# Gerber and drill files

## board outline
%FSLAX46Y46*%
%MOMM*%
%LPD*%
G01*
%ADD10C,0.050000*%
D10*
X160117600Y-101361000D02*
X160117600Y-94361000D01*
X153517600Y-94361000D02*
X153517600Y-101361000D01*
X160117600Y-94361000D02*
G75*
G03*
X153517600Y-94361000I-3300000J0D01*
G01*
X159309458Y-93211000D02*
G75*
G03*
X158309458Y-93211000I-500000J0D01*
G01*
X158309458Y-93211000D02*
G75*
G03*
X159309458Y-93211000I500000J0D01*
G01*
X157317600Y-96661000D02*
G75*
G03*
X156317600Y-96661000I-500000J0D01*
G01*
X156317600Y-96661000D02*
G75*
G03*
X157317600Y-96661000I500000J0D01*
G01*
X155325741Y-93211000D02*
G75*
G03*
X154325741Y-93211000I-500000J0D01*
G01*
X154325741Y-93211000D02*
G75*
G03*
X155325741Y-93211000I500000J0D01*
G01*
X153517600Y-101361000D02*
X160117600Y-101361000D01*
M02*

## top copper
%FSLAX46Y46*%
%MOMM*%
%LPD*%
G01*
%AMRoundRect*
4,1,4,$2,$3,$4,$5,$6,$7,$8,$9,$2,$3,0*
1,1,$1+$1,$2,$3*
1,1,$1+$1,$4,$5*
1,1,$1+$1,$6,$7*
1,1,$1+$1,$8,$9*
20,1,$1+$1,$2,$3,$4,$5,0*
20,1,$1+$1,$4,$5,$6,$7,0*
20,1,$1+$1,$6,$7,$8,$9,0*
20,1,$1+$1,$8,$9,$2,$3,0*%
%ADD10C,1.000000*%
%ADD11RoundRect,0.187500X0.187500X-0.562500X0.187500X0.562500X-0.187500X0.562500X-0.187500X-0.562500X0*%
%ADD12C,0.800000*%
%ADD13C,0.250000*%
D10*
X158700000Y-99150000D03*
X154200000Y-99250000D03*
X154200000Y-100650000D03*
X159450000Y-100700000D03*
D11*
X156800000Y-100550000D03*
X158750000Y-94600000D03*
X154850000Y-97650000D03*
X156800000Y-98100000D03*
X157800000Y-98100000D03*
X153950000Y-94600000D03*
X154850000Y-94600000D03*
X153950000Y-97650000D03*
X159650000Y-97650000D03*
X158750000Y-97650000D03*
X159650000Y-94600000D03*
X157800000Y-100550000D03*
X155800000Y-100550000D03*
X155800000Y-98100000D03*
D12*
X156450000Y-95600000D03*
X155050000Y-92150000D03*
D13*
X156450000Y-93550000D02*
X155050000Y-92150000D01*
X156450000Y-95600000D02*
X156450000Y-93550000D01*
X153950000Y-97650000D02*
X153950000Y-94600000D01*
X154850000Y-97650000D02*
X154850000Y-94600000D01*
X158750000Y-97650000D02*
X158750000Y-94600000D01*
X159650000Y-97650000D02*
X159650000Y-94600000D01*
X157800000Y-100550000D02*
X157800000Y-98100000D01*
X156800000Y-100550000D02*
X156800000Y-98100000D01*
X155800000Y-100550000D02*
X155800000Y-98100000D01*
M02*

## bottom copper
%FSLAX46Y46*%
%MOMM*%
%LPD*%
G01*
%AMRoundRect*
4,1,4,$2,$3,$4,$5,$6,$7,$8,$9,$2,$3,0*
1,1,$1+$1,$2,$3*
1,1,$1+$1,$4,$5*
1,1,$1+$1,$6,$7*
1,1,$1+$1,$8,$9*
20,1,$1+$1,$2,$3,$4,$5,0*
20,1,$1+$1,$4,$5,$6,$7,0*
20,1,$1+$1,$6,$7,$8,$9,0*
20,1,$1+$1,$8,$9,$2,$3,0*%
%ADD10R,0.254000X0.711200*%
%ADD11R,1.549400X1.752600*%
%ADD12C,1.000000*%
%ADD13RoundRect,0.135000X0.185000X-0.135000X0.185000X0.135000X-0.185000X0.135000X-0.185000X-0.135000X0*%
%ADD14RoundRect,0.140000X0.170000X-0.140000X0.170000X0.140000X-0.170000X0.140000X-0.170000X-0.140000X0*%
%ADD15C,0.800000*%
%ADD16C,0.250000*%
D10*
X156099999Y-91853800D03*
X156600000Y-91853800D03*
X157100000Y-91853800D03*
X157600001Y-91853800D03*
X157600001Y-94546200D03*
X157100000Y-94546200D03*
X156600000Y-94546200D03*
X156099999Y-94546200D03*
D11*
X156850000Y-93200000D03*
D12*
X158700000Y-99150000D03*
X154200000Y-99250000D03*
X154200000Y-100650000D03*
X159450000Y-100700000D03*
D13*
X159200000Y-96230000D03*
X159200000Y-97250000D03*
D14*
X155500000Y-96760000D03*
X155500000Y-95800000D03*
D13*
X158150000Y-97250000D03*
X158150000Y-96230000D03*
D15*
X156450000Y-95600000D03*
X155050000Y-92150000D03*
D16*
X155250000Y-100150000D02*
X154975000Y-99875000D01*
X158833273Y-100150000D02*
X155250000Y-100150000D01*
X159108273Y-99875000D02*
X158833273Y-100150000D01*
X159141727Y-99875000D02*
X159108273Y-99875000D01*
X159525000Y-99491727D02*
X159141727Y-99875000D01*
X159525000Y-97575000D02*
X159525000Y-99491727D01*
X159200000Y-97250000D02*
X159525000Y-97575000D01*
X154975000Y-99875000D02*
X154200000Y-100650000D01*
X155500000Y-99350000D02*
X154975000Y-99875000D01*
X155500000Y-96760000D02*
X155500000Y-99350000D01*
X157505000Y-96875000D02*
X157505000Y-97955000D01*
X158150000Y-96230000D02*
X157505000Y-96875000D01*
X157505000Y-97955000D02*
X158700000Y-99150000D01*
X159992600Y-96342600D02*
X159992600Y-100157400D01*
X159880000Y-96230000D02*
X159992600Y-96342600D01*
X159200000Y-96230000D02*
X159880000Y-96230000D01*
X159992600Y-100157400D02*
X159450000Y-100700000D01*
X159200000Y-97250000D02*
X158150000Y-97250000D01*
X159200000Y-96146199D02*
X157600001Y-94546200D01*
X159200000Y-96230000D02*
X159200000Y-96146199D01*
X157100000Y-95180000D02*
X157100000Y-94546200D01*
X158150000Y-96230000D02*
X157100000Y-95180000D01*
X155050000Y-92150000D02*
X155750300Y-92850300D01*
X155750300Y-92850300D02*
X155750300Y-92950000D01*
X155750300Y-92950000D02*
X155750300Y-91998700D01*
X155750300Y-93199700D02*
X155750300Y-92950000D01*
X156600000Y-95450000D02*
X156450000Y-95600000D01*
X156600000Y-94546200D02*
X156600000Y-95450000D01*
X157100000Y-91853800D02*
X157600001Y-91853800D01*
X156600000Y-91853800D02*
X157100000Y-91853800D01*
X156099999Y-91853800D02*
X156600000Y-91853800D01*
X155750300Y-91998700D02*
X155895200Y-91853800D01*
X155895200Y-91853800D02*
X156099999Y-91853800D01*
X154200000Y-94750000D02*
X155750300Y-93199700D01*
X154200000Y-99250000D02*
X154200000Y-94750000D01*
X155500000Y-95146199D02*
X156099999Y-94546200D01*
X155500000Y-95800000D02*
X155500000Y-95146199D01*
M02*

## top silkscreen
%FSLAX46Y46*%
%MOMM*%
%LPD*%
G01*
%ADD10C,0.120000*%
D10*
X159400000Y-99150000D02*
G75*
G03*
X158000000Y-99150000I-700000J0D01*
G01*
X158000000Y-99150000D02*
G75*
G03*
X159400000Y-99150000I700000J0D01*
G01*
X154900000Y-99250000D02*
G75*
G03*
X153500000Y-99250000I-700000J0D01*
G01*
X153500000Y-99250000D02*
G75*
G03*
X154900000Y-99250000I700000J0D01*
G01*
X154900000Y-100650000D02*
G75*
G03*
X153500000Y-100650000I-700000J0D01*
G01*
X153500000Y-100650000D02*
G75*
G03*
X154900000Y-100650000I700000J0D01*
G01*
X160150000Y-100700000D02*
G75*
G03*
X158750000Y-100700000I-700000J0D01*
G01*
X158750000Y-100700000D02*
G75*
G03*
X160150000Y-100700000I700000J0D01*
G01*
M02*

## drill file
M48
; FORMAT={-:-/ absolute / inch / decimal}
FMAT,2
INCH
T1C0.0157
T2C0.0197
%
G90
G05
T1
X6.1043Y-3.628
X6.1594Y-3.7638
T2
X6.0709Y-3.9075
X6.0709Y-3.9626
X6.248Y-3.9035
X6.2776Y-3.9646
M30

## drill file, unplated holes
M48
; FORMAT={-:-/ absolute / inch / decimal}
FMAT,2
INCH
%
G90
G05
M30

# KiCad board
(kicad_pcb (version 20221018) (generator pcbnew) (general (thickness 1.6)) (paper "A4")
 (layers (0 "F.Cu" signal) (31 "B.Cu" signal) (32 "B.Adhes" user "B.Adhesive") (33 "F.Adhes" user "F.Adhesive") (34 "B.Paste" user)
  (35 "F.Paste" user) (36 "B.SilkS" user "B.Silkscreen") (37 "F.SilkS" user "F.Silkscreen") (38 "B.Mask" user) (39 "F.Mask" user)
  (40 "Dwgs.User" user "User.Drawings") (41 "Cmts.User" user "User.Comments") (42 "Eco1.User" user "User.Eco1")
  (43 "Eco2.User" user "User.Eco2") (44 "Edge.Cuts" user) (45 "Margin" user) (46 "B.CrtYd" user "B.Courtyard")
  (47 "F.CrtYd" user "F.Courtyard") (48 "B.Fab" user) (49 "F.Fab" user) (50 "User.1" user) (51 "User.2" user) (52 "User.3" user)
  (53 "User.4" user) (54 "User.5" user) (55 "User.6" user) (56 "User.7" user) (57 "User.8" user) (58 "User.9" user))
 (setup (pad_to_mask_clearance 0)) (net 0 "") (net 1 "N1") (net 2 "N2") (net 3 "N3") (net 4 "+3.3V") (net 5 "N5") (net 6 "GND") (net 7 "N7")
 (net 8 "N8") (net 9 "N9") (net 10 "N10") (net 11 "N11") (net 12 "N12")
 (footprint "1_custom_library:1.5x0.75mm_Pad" (layer "F.Cu") (at 156.8 100.55 90)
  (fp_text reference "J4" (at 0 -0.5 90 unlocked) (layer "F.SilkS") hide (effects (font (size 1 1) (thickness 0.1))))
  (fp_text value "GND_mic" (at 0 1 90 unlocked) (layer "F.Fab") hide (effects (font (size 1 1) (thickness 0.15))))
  (pad "1" smd roundrect (at 0 0 90) (size 1.5 0.75) (layers "F.Cu" "F.Paste" "F.Mask") (roundrect_rratio 0.25) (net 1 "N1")
   (thermal_bridge_angle 45)))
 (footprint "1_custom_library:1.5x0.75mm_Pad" (layer "F.Cu") (at 158.75 94.6 90)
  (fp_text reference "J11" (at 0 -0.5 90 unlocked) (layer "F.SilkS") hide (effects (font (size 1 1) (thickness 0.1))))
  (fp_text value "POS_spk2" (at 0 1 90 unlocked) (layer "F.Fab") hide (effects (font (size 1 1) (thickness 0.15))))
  (pad "1" smd roundrect (at 0 0 90) (size 1.5 0.75) (layers "F.Cu" "F.Paste" "F.Mask") (roundrect_rratio 0.25) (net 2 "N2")
   (thermal_bridge_angle 45)))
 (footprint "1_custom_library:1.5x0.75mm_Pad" (layer "F.Cu") (at 154.85 97.65 90)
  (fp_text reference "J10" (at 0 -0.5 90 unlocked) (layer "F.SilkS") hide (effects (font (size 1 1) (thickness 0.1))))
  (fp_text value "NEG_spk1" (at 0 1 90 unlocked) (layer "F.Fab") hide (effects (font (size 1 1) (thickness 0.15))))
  (pad "1" smd roundrect (at 0 0 90) (size 1.5 0.75) (layers "F.Cu" "F.Paste" "F.Mask") (roundrect_rratio 0.25) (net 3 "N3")
   (thermal_bridge_angle 45)))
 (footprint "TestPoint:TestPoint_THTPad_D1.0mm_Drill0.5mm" (layer "F.Cu") (at 154.2 100.65 90)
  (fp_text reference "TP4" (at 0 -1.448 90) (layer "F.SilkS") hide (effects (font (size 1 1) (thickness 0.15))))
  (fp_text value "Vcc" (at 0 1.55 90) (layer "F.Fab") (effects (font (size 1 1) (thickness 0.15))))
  (fp_circle (center 0 0) (end 0 0.7) (stroke (width 0.12) (type solid)) (fill none) (layer "F.SilkS"))
  (pad "1" thru_hole circle (at 0 0 90) (size 1 1) (drill 0.5) (layers "*.Cu" "*.Mask") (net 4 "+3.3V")))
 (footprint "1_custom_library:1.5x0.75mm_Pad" (layer "F.Cu") (at 156.8 98.1 90)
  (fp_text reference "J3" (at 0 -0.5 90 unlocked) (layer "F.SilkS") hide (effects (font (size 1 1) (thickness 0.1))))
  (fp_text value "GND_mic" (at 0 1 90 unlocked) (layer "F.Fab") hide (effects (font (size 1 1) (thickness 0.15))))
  (pad "1" smd roundrect (at 0 0 90) (size 1.5 0.75) (layers "F.Cu" "F.Paste" "F.Mask") (roundrect_rratio 0.25) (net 1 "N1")
   (thermal_bridge_angle 45)))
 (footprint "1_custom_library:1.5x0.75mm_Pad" (layer "F.Cu") (at 157.8 98.1 90)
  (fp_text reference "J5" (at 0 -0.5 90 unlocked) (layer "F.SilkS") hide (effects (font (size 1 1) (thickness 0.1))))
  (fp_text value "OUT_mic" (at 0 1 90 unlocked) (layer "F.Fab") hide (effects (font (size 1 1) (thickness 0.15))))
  (pad "1" smd roundrect (at 0 0 90) (size 1.5 0.75) (layers "F.Cu" "F.Paste" "F.Mask") (roundrect_rratio 0.25) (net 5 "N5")
   (thermal_bridge_angle 45)))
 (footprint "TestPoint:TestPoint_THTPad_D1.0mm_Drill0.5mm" (layer "F.Cu") (at 154.2 99.25 90)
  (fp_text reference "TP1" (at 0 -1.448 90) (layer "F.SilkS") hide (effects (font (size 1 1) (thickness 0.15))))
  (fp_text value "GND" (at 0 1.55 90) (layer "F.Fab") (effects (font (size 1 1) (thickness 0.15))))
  (fp_circle (center 0 0) (end 0 0.7) (stroke (width 0.12) (type solid)) (fill none) (layer "F.SilkS"))
  (pad "1" thru_hole circle (at 0 0 90) (size 1 1) (drill 0.5) (layers "*.Cu" "*.Mask") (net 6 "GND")))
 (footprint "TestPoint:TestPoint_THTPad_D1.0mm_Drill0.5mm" (layer "F.Cu") (at 158.7 99.15 90)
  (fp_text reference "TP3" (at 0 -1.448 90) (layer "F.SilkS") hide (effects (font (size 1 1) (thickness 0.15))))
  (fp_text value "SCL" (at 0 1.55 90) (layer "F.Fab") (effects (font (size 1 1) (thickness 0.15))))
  (fp_circle (center 0 0) (end 0 0.7) (stroke (width 0.12) (type solid)) (fill none) (layer "F.SilkS"))
  (pad "1" thru_hole circle (at 0 0 90) (size 1 1) (drill 0.5) (layers "*.Cu" "*.Mask") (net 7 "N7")))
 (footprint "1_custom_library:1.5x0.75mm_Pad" (layer "F.Cu") (at 153.95 94.6 90)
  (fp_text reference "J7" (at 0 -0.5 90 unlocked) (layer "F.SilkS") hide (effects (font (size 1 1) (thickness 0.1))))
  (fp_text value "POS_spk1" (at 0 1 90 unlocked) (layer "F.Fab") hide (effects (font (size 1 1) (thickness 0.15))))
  (pad "1" smd roundrect (at 0 0 90) (size 1.5 0.75) (layers "F.Cu" "F.Paste" "F.Mask") (roundrect_rratio 0.25) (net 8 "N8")
   (thermal_bridge_angle 45)))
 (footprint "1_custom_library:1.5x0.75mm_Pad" (layer "F.Cu") (at 154.85 94.6 90)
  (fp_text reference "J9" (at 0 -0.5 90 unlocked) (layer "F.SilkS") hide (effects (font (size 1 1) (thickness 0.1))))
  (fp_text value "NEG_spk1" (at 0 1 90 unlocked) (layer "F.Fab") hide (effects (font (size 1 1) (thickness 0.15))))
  (pad "1" smd roundrect (at 0 0 90) (size 1.5 0.75) (layers "F.Cu" "F.Paste" "F.Mask") (roundrect_rratio 0.25) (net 3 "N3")
   (thermal_bridge_angle 45)))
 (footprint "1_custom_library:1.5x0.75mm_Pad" (layer "F.Cu") (at 153.95 97.65 90)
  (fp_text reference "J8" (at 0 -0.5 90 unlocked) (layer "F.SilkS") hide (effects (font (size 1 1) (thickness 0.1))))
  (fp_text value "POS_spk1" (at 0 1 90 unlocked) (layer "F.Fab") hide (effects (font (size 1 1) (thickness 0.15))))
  (pad "1" smd roundrect (at 0 0 90) (size 1.5 0.75) (layers "F.Cu" "F.Paste" "F.Mask") (roundrect_rratio 0.25) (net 8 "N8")
   (thermal_bridge_angle 45)))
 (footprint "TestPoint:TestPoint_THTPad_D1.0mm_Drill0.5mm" (layer "F.Cu") (at 159.45 100.7 90)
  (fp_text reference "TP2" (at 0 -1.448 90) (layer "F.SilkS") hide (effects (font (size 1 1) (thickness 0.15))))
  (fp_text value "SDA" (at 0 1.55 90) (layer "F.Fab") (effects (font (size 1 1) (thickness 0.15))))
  (fp_circle (center 0 0) (end 0 0.7) (stroke (width 0.12) (type solid)) (fill none) (layer "F.SilkS"))
  (pad "1" thru_hole circle (at 0 0 90) (size 1 1) (drill 0.5) (layers "*.Cu" "*.Mask") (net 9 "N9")))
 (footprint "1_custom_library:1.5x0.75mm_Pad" (layer "F.Cu") (at 159.65 97.65 90)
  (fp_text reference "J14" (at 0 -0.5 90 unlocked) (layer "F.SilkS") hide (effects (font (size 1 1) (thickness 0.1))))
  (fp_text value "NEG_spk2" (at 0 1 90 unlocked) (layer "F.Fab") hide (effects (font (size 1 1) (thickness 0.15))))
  (pad "1" smd roundrect (at 0 0 90) (size 1.5 0.75) (layers "F.Cu" "F.Paste" "F.Mask") (roundrect_rratio 0.25) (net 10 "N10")
   (thermal_bridge_angle 45)))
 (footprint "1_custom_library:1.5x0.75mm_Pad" (layer "F.Cu") (at 158.75 97.65 90)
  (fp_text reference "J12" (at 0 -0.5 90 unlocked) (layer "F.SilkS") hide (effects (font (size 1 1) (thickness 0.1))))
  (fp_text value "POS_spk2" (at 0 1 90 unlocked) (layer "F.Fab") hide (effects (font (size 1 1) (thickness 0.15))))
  (pad "1" smd roundrect (at 0 0 90) (size 1.5 0.75) (layers "F.Cu" "F.Paste" "F.Mask") (roundrect_rratio 0.25) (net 2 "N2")
   (thermal_bridge_angle 45)))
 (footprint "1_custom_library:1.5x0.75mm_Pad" (layer "F.Cu") (at 159.65 94.6 90)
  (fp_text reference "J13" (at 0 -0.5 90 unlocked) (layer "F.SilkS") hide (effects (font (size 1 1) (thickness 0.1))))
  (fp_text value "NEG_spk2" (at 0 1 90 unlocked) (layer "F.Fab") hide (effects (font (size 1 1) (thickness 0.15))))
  (pad "1" smd roundrect (at 0 0 90) (size 1.5 0.75) (layers "F.Cu" "F.Paste" "F.Mask") (roundrect_rratio 0.25) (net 10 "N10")
   (thermal_bridge_angle 45)))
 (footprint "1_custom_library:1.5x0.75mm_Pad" (layer "F.Cu") (at 157.8 100.55 90)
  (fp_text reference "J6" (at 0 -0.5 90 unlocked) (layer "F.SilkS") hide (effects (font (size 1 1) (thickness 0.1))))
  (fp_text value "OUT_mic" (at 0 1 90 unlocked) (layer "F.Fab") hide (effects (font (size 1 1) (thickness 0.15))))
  (pad "1" smd roundrect (at 0 0 90) (size 1.5 0.75) (layers "F.Cu" "F.Paste" "F.Mask") (roundrect_rratio 0.25) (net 5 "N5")
   (thermal_bridge_angle 45)))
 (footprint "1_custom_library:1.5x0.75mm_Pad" (layer "F.Cu") (at 155.8 100.55 90)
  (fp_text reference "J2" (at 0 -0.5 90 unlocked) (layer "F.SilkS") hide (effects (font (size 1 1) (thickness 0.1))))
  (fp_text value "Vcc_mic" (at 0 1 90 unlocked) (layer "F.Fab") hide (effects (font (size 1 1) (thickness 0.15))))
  (pad "1" smd roundrect (at 0 0 90) (size 1.5 0.75) (layers "F.Cu" "F.Paste" "F.Mask") (roundrect_rratio 0.25) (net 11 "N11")
   (thermal_bridge_angle 45)))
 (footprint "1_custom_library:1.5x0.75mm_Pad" (layer "F.Cu") (at 155.8 98.1 90)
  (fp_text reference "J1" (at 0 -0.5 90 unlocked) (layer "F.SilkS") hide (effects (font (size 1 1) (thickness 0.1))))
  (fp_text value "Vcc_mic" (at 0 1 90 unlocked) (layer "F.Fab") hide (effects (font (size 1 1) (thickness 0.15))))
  (pad "1" smd roundrect (at 0 0 90) (size 1.5 0.75) (layers "F.Cu" "F.Paste" "F.Mask") (roundrect_rratio 0.25) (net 11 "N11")
   (thermal_bridge_angle 45)))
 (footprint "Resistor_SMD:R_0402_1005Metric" (layer "B.Cu") (at 159.2 96.74 90)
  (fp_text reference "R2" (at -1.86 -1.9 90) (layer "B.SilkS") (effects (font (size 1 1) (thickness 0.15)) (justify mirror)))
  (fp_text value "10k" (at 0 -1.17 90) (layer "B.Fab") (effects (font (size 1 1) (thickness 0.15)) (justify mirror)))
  (pad "1" smd roundrect (at -0.51 0 90) (size 0.54 0.64) (layers "B.Cu" "B.Paste" "B.Mask") (roundrect_rratio 0.25) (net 4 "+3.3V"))
  (pad "2" smd roundrect (at 0.51 0 90) (size 0.54 0.64) (layers "B.Cu" "B.Paste" "B.Mask") (roundrect_rratio 0.25) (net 9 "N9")))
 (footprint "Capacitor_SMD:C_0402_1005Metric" (layer "B.Cu") (at 155.5 96.28 90)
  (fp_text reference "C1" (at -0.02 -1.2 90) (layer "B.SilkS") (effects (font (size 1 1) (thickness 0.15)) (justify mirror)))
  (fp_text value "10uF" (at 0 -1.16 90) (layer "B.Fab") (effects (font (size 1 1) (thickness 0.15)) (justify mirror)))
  (pad "1" smd roundrect (at -0.48 0 90) (size 0.56 0.62) (layers "B.Cu" "B.Paste" "B.Mask") (roundrect_rratio 0.25) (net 4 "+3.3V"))
  (pad "2" smd roundrect (at 0.48 0 90) (size 0.56 0.62) (layers "B.Cu" "B.Paste" "B.Mask") (roundrect_rratio 0.25) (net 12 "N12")))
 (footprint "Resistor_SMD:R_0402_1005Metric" (layer "B.Cu") (at 158.15 96.74 90)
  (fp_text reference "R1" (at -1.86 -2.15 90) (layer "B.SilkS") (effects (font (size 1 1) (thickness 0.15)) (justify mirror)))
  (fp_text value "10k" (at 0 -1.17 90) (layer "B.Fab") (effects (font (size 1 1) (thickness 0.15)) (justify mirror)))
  (pad "1" smd roundrect (at -0.51 0 90) (size 0.54 0.64) (layers "B.Cu" "B.Paste" "B.Mask") (roundrect_rratio 0.25) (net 4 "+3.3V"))
  (pad "2" smd roundrect (at 0.51 0 90) (size 0.54 0.64) (layers "B.Cu" "B.Paste" "B.Mask") (roundrect_rratio 0.25) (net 7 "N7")))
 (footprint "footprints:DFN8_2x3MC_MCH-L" (layer "B.Cu") (at 156.85 93.2 -90)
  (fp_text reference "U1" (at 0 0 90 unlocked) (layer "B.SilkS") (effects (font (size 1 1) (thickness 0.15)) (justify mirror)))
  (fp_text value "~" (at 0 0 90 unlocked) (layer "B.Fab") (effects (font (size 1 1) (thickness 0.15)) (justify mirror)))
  (pad "1" smd rect (at -1.3462 0.750001 270) (size 0.7112 0.254) (layers "B.Cu" "B.Paste" "B.Mask") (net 6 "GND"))
  (pad "2" smd rect (at -1.3462 0.25 270) (size 0.7112 0.254) (layers "B.Cu" "B.Paste" "B.Mask") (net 6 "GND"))
  (pad "3" smd rect (at -1.3462 -0.25 270) (size 0.7112 0.254) (layers "B.Cu" "B.Paste" "B.Mask") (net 6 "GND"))
  (pad "4" smd rect (at -1.3462 -0.750001 270) (size 0.7112 0.254) (layers "B.Cu" "B.Paste" "B.Mask") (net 6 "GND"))
  (pad "5" smd rect (at 1.3462 -0.750001 270) (size 0.7112 0.254) (layers "B.Cu" "B.Paste" "B.Mask") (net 9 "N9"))
  (pad "6" smd rect (at 1.3462 -0.25 270) (size 0.7112 0.254) (layers "B.Cu" "B.Paste" "B.Mask") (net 7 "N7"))
  (pad "7" smd rect (at 1.3462 0.25 270) (size 0.7112 0.254) (layers "B.Cu" "B.Paste" "B.Mask") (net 6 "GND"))
  (pad "8" smd rect (at 1.3462 0.750001 270) (size 0.7112 0.254) (layers "B.Cu" "B.Paste" "B.Mask") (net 12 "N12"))
  (pad "9" smd rect (at 0 0 270) (size 1.7526 1.5494) (layers "B.Cu" "B.Paste" "B.Mask")))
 (gr_line (start 160.1176 101.361) (end 160.1176 94.361) (stroke (width 0.05) (type solid)) (layer "Edge.Cuts"))
 (gr_line (start 153.5176 94.361) (end 153.5176 101.361) (stroke (width 0.05) (type solid)) (layer "Edge.Cuts"))
 (gr_arc (start 153.5176 94.361) (mid 156.8176 91.061) (end 160.1176 94.361) (stroke (width 0.05) (type solid)) (layer "Edge.Cuts"))
 (gr_circle (center 158.809458 93.211) (end 159.309458 93.211) (stroke (width 0.05) (type solid)) (fill none) (layer "Edge.Cuts"))
 (gr_circle (center 156.8176 96.661) (end 157.3176 96.661) (stroke (width 0.05) (type solid)) (fill none) (layer "Edge.Cuts"))
 (gr_circle (center 154.825741 93.211) (end 155.325741 93.211) (stroke (width 0.05) (type solid)) (fill none) (layer "Edge.Cuts"))
 (gr_line (start 153.5176 101.361) (end 160.1176 101.361) (stroke (width 0.05) (type solid)) (layer "Edge.Cuts"))
 (segment (start 159.108273 99.875) (end 158.833273 100.15) (width 0.25) (layer "B.Cu") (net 4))
 (segment (start 158.833273 100.15) (end 155.25 100.15) (width 0.25) (layer "B.Cu") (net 4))
 (segment (start 159.2 97.25) (end 158.15 97.25) (width 0.25) (layer "B.Cu") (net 4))
 (segment (start 159.2 97.25) (end 159.525 97.575) (width 0.25) (layer "B.Cu") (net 4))
 (segment (start 154.975 99.875) (end 154.2 100.65) (width 0.25) (layer "B.Cu") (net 4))
 (segment (start 159.525 99.491727) (end 159.141727 99.875) (width 0.25) (layer "B.Cu") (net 4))
 (segment (start 159.525 97.575) (end 159.525 99.491727) (width 0.25) (layer "B.Cu") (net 4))
 (segment (start 159.141727 99.875) (end 159.108273 99.875) (width 0.25) (layer "B.Cu") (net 4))
 (segment (start 155.5 96.76) (end 155.5 99.35) (width 0.25) (layer "B.Cu") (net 4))
 (segment (start 155.25 100.15) (end 154.975 99.875) (width 0.25) (layer "B.Cu") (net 4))
 (segment (start 155.5 99.35) (end 154.975 99.875) (width 0.25) (layer "B.Cu") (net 4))
 (segment (start 155.5 95.146199) (end 156.099999 94.5462) (width 0.25) (layer "B.Cu") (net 12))
 (segment (start 155.5 95.8) (end 155.5 95.146199) (width 0.25) (layer "B.Cu") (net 12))
 (segment (start 156.45 93.55) (end 155.05 92.15) (width 0.25) (layer "F.Cu") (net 6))
 (segment (start 156.45 95.6) (end 156.45 93.55) (width 0.25) (layer "F.Cu") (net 6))
 (via (at 156.45 95.6) (size 0.8) (drill 0.4) (layers "F.Cu" "B.Cu") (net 6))
 (via (at 155.05 92.15) (size 0.8) (drill 0.4) (layers "F.Cu" "B.Cu") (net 6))
 (segment (start 157.1 91.8538) (end 157.600001 91.8538) (width 0.25) (layer "B.Cu") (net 6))
 (segment (start 155.7503 91.9987) (end 155.8952 91.8538) (width 0.25) (layer "B.Cu") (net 6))
 (segment (start 155.7503 92.8503) (end 155.7503 92.95) (width 0.25) (layer "B.Cu") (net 6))
 (segment (start 156.6 94.5462) (end 156.6 95.45) (width 0.25) (layer "B.Cu") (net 6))
 (segment (start 156.6 95.45) (end 156.45 95.6) (width 0.25) (layer "B.Cu") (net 6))
 (segment (start 156.6 91.8538) (end 157.1 91.8538) (width 0.25) (layer "B.Cu") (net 6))
 (segment (start 155.7503 92.95) (end 155.7503 91.9987) (width 0.25) (layer "B.Cu") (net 6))
 (segment (start 156.099999 91.8538) (end 156.6 91.8538) (width 0.25) (layer "B.Cu") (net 6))
 (segment (start 154.2 94.75) (end 155.7503 93.1997) (width 0.25) (layer "B.Cu") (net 6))
 (segment (start 154.2 99.25) (end 154.2 94.75) (width 0.25) (layer "B.Cu") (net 6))
 (segment (start 155.05 92.15) (end 155.7503 92.8503) (width 0.25) (layer "B.Cu") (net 6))
 (segment (start 155.7503 93.1997) (end 155.7503 92.95) (width 0.25) (layer "B.Cu") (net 6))
 (segment (start 155.8952 91.8538) (end 156.099999 91.8538) (width 0.25) (layer "B.Cu") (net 6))
 (segment (start 157.1 95.18) (end 157.1 94.5462) (width 0.25) (layer "B.Cu") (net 7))
 (segment (start 157.505 96.875) (end 157.505 97.955) (width 0.25) (layer "B.Cu") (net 7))
 (segment (start 158.15 96.23) (end 157.505 96.875) (width 0.25) (layer "B.Cu") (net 7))
 (segment (start 158.15 96.23) (end 157.1 95.18) (width 0.25) (layer "B.Cu") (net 7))
 (segment (start 157.505 97.955) (end 158.7 99.15) (width 0.25) (layer "B.Cu") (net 7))
 (segment (start 159.9926 96.3426) (end 159.9926 100.1574) (width 0.25) (layer "B.Cu") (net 9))
 (segment (start 159.2 96.23) (end 159.88 96.23) (width 0.25) (layer "B.Cu") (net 9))
 (segment (start 159.9926 100.1574) (end 159.45 100.7) (width 0.25) (layer "B.Cu") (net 9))
 (segment (start 159.88 96.23) (end 159.9926 96.3426) (width 0.25) (layer "B.Cu") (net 9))
 (segment (start 159.2 96.146199) (end 157.600001 94.5462) (width 0.25) (layer "B.Cu") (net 9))
 (segment (start 159.2 96.23) (end 159.2 96.146199) (width 0.25) (layer "B.Cu") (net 9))
 (segment (start 155.8 100.55) (end 155.8 98.1) (width 0.25) (layer "F.Cu") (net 11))
 (segment (start 156.8 100.55) (end 156.8 98.1) (width 0.25) (layer "F.Cu") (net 1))
 (segment (start 157.8 100.55) (end 157.8 98.1) (width 0.25) (layer "F.Cu") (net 5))
 (segment (start 153.95 97.65) (end 153.95 94.6) (width 0.25) (layer "F.Cu") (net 8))
 (segment (start 154.85 97.65) (end 154.85 94.6) (width 0.25) (layer "F.Cu") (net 3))
 (segment (start 158.75 97.65) (end 158.75 94.6) (width 0.25) (layer "F.Cu") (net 2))
 (segment (start 159.65 97.65) (end 159.65 94.6) (width 0.25) (layer "F.Cu") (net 10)))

